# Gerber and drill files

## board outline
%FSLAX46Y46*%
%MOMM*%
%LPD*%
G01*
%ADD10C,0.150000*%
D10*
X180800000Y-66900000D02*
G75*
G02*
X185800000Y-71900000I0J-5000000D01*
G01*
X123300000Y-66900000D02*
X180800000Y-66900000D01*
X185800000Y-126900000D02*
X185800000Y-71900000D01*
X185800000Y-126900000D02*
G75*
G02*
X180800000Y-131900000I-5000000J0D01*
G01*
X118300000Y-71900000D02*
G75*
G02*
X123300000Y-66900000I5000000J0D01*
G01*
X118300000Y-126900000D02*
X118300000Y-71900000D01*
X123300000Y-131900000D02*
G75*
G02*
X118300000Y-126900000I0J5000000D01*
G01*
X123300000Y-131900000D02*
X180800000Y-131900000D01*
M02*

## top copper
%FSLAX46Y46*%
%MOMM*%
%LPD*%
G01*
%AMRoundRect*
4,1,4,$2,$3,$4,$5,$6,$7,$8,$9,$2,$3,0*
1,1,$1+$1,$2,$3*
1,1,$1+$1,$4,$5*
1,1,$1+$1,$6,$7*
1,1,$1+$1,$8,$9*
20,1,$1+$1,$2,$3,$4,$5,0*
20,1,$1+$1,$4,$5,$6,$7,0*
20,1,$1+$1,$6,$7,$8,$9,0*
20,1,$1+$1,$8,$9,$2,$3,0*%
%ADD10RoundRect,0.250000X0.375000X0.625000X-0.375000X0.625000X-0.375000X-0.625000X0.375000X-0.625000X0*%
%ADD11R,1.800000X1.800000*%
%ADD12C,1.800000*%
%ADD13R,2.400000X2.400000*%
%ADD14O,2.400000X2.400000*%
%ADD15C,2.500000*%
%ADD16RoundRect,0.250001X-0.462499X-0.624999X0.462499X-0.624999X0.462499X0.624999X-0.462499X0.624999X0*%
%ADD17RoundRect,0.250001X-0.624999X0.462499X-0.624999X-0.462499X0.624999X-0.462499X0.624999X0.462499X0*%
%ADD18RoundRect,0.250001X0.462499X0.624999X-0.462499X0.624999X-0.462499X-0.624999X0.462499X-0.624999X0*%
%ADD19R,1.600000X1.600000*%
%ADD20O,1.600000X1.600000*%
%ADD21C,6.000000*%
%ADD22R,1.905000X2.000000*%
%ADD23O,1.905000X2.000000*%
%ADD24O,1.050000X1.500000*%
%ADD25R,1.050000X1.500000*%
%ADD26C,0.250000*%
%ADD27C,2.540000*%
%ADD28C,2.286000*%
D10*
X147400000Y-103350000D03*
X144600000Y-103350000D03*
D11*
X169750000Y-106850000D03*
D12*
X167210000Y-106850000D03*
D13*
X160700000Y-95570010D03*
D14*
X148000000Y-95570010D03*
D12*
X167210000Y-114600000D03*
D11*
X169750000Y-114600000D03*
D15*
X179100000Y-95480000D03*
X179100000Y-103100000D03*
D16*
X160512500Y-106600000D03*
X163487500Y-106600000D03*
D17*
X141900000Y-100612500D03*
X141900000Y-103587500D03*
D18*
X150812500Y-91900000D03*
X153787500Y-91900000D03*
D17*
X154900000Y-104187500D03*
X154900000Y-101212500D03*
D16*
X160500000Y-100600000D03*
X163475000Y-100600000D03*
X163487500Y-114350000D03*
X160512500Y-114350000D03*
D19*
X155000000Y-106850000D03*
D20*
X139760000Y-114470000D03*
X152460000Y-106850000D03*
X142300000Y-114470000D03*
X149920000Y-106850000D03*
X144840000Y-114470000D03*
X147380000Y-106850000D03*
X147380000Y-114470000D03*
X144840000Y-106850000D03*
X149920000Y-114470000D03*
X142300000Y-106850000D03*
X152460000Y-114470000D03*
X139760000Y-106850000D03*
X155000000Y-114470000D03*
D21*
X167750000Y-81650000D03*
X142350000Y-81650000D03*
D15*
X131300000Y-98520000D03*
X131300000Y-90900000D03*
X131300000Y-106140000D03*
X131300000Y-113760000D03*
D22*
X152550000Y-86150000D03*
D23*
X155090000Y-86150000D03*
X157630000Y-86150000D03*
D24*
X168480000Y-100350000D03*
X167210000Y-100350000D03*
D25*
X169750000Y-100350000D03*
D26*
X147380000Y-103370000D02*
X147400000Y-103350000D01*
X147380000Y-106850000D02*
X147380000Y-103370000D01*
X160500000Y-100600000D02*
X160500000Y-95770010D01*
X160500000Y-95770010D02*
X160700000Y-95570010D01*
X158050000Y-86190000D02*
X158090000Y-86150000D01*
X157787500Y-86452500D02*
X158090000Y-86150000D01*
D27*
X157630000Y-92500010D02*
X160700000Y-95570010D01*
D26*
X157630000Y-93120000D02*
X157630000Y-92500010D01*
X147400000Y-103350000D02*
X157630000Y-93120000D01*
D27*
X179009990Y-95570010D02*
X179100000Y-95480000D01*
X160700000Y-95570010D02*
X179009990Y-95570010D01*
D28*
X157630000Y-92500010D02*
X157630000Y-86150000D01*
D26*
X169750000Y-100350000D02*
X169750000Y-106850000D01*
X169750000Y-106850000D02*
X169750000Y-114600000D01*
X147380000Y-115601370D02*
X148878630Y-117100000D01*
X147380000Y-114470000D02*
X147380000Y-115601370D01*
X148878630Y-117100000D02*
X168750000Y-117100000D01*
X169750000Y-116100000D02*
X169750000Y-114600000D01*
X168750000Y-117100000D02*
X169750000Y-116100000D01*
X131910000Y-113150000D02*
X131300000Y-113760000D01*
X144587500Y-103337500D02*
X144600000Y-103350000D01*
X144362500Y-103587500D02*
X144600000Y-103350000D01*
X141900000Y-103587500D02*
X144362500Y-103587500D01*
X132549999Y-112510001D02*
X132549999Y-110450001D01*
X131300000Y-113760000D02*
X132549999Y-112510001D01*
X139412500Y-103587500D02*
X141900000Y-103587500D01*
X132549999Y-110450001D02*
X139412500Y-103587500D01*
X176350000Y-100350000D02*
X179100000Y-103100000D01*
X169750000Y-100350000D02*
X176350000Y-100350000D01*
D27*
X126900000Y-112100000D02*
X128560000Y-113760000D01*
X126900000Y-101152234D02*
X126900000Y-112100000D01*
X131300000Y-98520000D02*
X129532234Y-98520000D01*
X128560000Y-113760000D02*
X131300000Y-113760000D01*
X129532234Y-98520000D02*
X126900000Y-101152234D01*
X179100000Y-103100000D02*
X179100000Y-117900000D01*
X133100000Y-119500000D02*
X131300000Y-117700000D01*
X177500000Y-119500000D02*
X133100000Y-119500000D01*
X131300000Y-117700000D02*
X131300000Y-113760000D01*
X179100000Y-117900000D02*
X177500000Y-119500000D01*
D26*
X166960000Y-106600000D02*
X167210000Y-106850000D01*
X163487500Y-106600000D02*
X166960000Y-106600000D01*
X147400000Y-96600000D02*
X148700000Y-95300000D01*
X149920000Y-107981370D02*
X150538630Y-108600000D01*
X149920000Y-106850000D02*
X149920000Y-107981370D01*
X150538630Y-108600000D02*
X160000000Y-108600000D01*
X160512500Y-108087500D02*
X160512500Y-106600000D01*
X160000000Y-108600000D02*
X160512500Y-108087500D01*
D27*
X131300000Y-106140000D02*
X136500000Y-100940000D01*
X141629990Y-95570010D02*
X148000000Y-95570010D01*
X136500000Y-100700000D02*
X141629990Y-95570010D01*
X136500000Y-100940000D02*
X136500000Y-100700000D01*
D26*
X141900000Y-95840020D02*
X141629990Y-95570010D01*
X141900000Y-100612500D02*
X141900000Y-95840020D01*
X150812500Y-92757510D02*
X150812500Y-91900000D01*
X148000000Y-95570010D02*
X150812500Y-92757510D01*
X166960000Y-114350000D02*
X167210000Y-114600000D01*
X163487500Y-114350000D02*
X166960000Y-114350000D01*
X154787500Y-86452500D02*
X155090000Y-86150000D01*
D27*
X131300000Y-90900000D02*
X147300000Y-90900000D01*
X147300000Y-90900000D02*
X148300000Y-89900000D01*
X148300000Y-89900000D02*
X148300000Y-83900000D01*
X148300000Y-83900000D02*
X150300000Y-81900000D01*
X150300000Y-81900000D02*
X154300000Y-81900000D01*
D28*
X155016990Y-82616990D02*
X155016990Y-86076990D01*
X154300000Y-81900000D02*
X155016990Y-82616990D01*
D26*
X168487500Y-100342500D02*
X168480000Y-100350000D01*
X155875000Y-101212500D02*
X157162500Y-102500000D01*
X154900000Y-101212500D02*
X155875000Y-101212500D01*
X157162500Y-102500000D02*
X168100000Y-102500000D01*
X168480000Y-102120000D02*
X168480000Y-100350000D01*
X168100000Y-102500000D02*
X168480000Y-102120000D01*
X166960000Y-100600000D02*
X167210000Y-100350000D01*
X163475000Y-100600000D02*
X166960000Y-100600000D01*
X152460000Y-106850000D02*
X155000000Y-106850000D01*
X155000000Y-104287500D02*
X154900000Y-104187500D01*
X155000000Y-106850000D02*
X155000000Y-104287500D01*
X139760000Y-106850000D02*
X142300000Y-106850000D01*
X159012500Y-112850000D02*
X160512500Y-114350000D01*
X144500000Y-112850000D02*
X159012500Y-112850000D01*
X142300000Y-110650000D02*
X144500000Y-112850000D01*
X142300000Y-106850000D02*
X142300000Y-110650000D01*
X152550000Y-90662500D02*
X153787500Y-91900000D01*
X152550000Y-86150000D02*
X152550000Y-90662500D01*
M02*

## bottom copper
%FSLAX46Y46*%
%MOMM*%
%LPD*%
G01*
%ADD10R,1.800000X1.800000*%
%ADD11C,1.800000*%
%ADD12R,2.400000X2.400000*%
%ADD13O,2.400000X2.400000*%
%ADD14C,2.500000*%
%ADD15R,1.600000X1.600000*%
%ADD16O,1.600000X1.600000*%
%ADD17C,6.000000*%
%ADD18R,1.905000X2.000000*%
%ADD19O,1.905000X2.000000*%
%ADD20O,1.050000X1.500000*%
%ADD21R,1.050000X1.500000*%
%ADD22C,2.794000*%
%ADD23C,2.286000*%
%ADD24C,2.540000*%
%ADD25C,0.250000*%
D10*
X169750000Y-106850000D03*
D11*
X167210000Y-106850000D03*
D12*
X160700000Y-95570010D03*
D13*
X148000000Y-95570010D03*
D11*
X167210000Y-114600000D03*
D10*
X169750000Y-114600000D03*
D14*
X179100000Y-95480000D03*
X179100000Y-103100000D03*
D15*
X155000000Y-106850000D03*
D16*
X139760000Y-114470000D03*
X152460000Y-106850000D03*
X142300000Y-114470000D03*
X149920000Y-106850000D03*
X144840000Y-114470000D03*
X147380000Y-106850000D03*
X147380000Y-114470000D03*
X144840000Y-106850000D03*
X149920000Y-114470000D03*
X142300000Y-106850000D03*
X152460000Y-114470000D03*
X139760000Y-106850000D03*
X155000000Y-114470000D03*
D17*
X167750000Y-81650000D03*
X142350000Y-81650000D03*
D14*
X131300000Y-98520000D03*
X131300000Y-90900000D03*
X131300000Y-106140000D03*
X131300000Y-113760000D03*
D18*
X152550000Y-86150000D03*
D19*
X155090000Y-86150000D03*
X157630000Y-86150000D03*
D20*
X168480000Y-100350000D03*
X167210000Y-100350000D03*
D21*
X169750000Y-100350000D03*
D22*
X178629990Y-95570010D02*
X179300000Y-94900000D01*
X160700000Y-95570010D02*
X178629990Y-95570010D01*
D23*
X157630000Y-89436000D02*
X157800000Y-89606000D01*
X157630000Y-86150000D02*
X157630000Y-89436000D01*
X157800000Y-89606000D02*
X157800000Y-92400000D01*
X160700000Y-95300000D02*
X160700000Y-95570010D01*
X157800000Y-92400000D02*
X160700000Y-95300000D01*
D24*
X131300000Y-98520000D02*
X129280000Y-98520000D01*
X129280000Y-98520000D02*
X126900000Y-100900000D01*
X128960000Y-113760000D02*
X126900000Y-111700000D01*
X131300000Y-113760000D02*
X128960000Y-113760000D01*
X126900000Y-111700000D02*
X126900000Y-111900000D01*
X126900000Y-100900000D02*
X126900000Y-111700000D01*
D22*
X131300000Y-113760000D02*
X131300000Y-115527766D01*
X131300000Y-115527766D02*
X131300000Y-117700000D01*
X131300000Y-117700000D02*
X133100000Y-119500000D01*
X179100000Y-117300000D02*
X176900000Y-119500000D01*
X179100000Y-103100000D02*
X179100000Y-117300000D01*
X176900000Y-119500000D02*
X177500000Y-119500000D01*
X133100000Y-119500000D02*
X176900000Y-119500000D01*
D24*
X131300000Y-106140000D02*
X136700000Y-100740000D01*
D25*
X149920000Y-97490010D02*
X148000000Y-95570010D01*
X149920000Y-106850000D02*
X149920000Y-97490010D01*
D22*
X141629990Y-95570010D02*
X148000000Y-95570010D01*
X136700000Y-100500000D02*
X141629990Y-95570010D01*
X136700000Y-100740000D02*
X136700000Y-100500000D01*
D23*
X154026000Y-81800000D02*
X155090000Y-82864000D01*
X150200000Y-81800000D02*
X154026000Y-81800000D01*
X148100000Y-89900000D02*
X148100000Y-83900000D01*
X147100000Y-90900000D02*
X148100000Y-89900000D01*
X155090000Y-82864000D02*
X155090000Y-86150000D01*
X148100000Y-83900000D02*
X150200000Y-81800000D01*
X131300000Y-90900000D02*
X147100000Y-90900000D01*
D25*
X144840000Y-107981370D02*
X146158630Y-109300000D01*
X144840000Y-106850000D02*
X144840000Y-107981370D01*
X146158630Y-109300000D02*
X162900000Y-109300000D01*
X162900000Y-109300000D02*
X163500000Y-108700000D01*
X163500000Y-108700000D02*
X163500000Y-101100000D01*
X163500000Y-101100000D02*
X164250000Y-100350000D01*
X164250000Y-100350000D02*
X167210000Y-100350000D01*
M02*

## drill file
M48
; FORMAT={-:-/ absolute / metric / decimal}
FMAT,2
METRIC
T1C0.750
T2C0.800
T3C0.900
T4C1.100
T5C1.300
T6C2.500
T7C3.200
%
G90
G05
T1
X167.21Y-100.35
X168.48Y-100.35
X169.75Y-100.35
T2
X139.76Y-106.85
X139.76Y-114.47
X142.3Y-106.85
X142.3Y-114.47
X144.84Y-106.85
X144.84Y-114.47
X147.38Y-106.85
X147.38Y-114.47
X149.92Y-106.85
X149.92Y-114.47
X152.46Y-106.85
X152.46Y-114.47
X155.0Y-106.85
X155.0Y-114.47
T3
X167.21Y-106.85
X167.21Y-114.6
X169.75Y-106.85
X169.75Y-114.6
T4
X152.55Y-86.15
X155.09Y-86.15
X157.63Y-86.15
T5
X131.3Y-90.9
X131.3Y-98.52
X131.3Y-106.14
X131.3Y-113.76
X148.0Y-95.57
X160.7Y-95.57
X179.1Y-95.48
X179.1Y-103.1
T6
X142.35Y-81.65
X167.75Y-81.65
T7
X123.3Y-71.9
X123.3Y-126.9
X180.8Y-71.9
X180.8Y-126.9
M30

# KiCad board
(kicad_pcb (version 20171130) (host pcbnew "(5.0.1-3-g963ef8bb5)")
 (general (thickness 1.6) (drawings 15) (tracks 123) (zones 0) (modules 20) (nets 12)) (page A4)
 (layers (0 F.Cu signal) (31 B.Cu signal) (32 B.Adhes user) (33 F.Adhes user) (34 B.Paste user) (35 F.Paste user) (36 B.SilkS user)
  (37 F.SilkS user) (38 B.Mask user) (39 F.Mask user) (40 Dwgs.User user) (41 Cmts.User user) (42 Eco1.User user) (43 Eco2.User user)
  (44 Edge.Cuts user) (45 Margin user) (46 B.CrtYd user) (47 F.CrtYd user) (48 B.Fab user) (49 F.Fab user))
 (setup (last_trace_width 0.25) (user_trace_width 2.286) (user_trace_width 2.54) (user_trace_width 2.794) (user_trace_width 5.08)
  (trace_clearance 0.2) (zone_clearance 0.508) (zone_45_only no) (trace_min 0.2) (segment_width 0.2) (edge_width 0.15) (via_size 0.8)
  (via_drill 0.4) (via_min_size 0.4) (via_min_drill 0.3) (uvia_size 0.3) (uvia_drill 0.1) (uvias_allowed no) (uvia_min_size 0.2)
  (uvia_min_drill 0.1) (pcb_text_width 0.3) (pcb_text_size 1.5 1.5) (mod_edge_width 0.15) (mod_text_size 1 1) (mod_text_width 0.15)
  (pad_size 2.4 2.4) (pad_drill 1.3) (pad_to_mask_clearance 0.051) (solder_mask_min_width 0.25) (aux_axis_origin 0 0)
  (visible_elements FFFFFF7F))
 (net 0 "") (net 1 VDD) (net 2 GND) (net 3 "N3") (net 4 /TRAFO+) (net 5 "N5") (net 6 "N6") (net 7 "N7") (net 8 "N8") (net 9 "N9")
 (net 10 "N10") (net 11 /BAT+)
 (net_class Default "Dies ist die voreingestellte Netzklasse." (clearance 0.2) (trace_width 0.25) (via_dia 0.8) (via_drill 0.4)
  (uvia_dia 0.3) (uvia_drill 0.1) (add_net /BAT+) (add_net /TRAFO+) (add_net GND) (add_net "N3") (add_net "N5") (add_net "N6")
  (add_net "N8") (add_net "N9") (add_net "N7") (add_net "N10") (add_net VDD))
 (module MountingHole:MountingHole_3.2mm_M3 (layer F.Cu) (at 180.8 126.9)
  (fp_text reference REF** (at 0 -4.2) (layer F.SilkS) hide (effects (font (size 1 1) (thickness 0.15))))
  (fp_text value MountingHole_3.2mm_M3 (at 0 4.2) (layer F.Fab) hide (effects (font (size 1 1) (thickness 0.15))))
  (pad 1 np_thru_hole circle (at 0 0) (size 3.2 3.2) (drill 3.2) (layers *.Cu *.Mask)))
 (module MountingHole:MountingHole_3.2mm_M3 (layer F.Cu) (at 180.8 71.9)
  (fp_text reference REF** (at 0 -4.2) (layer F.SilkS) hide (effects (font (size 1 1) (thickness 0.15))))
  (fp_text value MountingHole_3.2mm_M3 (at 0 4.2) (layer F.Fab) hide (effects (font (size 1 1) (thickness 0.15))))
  (pad 1 np_thru_hole circle (at 0 0) (size 3.2 3.2) (drill 3.2) (layers *.Cu *.Mask)))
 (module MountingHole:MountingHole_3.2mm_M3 (layer F.Cu) (at 123.3 71.9)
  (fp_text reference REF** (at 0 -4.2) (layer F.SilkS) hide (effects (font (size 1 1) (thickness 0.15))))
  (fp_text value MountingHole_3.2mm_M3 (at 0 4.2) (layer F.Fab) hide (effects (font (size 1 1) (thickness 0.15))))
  (pad 1 np_thru_hole circle (at 0 0) (size 3.2 3.2) (drill 3.2) (layers *.Cu *.Mask)))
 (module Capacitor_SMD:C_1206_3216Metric (layer F.Cu) (at 146 103.35 180)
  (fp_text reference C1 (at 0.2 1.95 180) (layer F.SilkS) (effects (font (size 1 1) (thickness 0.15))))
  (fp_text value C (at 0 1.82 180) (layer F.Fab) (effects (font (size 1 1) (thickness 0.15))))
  (pad 1 smd roundrect (at -1.4 0 180) (size 1.25 1.75) (layers F.Cu F.Paste F.Mask) (roundrect_rratio 0.2) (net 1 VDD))
  (pad 2 smd roundrect (at 1.4 0 180) (size 1.25 1.75) (layers F.Cu F.Paste F.Mask) (roundrect_rratio 0.2) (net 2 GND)))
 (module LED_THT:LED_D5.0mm (layer F.Cu) (at 169.75 106.85 180)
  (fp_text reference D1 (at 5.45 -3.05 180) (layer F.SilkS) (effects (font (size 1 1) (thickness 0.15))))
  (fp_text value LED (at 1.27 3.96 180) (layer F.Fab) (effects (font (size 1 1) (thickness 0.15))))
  (pad 1 thru_hole rect (at 0 0 180) (size 1.8 1.8) (drill 0.9) (layers *.Cu *.Mask) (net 2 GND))
  (pad 2 thru_hole circle (at 2.54 0 180) (size 1.8 1.8) (drill 0.9) (layers *.Cu *.Mask) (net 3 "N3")))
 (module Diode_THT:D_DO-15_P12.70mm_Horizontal (layer F.Cu) (at 160.7 95.57001 180)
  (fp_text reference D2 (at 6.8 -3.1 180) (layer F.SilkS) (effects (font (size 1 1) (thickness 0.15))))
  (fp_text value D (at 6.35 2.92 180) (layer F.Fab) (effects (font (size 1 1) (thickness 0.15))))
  (pad 1 thru_hole rect (at 0 0 180) (size 2.4 2.4) (drill 1.3) (layers *.Cu *.Mask) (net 1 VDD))
  (pad 2 thru_hole oval (at 12.7 0 180) (size 2.4 2.4) (drill 1.3) (layers *.Cu *.Mask) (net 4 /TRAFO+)))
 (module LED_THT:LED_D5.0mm (layer F.Cu) (at 169.75 114.6 180)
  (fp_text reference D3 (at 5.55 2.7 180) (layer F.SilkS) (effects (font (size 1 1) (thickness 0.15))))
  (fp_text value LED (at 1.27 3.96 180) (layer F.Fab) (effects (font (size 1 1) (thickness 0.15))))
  (pad 2 thru_hole circle (at 2.54 0 180) (size 1.8 1.8) (drill 0.9) (layers *.Cu *.Mask) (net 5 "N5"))
  (pad 1 thru_hole rect (at 0 0 180) (size 1.8 1.8) (drill 0.9) (layers *.Cu *.Mask) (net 2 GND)))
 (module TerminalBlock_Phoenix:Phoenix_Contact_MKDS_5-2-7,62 (layer F.Cu) (at 179.1 103.1 90)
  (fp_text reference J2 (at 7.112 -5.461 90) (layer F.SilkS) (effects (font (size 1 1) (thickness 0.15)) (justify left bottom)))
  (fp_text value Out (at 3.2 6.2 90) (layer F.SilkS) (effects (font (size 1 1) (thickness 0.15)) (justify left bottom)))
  (pad 2 thru_hole circle (at 7.62 0 90) (size 2.5 2.5) (drill 1.3) (layers *.Cu *.Mask) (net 1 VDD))
  (pad 1 thru_hole circle (at 0 0 90) (size 2.5 2.5) (drill 1.3) (layers *.Cu *.Mask) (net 2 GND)))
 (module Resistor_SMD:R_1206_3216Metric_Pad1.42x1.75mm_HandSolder (layer F.Cu) (at 162 106.6)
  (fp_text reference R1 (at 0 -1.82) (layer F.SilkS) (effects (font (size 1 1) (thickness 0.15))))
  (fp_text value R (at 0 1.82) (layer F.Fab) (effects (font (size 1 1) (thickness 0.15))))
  (pad 1 smd roundrect (at -1.4875 0) (size 1.425 1.75) (layers F.Cu F.Paste F.Mask) (roundrect_rratio 0.175439) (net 4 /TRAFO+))
  (pad 2 smd roundrect (at 1.4875 0) (size 1.425 1.75) (layers F.Cu F.Paste F.Mask) (roundrect_rratio 0.175439) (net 3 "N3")))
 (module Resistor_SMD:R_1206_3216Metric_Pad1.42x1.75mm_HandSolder (layer F.Cu) (at 141.9 102.1 270)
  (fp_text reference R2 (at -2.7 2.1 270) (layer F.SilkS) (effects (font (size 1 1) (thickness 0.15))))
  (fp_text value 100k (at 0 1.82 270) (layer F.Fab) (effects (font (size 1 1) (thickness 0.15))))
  (pad 1 smd roundrect (at -1.4875 0 270) (size 1.425 1.75) (layers F.Cu F.Paste F.Mask) (roundrect_rratio 0.175439) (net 4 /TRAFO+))
  (pad 2 smd roundrect (at 1.4875 0 270) (size 1.425 1.75) (layers F.Cu F.Paste F.Mask) (roundrect_rratio 0.175439) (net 2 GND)))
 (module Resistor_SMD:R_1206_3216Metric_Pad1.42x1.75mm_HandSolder (layer F.Cu) (at 152.3 91.9 180)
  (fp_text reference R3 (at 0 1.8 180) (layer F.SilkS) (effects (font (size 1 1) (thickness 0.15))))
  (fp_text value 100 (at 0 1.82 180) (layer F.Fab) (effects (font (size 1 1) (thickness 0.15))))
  (pad 2 smd roundrect (at 1.4875 0 180) (size 1.425 1.75) (layers F.Cu F.Paste F.Mask) (roundrect_rratio 0.175439) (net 4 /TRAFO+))
  (pad 1 smd roundrect (at -1.4875 0 180) (size 1.425 1.75) (layers F.Cu F.Paste F.Mask) (roundrect_rratio 0.175439) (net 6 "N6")))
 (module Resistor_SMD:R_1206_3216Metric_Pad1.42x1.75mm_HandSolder (layer F.Cu) (at 154.9 102.7 270)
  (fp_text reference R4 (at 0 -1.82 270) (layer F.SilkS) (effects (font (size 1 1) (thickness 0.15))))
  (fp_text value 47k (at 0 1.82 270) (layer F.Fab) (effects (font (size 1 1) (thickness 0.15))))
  (pad 2 smd roundrect (at 1.4875 0 270) (size 1.425 1.75) (layers F.Cu F.Paste F.Mask) (roundrect_rratio 0.175439) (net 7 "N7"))
  (pad 1 smd roundrect (at -1.4875 0 270) (size 1.425 1.75) (layers F.Cu F.Paste F.Mask) (roundrect_rratio 0.175439) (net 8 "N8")))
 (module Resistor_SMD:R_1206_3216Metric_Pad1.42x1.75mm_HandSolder (layer F.Cu) (at 161.9875 100.6)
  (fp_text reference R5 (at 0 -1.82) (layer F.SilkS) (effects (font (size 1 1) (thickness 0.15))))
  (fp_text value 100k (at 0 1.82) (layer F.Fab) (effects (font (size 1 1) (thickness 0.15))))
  (pad 1 smd roundrect (at -1.4875 0) (size 1.425 1.75) (layers F.Cu F.Paste F.Mask) (roundrect_rratio 0.175439) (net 1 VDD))
  (pad 2 smd roundrect (at 1.4875 0) (size 1.425 1.75) (layers F.Cu F.Paste F.Mask) (roundrect_rratio 0.175439) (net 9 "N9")))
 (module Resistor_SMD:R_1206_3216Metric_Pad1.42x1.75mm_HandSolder (layer F.Cu) (at 162 114.35)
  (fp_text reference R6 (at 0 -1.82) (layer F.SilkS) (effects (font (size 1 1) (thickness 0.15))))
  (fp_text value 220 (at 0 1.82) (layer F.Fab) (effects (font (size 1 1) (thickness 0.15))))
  (pad 2 smd roundrect (at 1.4875 0) (size 1.425 1.75) (layers F.Cu F.Paste F.Mask) (roundrect_rratio 0.175439) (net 5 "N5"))
  (pad 1 smd roundrect (at -1.4875 0) (size 1.425 1.75) (layers F.Cu F.Paste F.Mask) (roundrect_rratio 0.175439) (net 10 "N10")))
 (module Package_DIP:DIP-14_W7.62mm (layer F.Cu) (at 155 106.85 270)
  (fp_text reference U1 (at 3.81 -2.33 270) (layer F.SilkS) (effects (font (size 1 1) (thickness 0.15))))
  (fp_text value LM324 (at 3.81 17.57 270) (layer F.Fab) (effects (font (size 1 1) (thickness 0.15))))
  (pad 1 thru_hole rect (at 0 0 270) (size 1.6 1.6) (drill 0.8) (layers *.Cu *.Mask) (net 7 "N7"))
  (pad 8 thru_hole oval (at 7.62 15.24 270) (size 1.6 1.6) (drill 0.8) (layers *.Cu *.Mask))
  (pad 2 thru_hole oval (at 0 2.54 270) (size 1.6 1.6) (drill 0.8) (layers *.Cu *.Mask) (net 7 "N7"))
  (pad 9 thru_hole oval (at 7.62 12.7 270) (size 1.6 1.6) (drill 0.8) (layers *.Cu *.Mask))
  (pad 3 thru_hole oval (at 0 5.08 270) (size 1.6 1.6) (drill 0.8) (layers *.Cu *.Mask) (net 4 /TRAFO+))
  (pad 10 thru_hole oval (at 7.62 10.16 270) (size 1.6 1.6) (drill 0.8) (layers *.Cu *.Mask))
  (pad 4 thru_hole oval (at 0 7.62 270) (size 1.6 1.6) (drill 0.8) (layers *.Cu *.Mask) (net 1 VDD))
  (pad 11 thru_hole oval (at 7.62 7.62 270) (size 1.6 1.6) (drill 0.8) (layers *.Cu *.Mask) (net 2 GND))
  (pad 5 thru_hole oval (at 0 10.16 270) (size 1.6 1.6) (drill 0.8) (layers *.Cu *.Mask) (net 9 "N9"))
  (pad 12 thru_hole oval (at 7.62 5.08 270) (size 1.6 1.6) (drill 0.8) (layers *.Cu *.Mask))
  (pad 6 thru_hole oval (at 0 12.7 270) (size 1.6 1.6) (drill 0.8) (layers *.Cu *.Mask) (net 10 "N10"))
  (pad 13 thru_hole oval (at 7.62 2.54 270) (size 1.6 1.6) (drill 0.8) (layers *.Cu *.Mask))
  (pad 7 thru_hole oval (at 0 15.24 270) (size 1.6 1.6) (drill 0.8) (layers *.Cu *.Mask) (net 10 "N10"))
  (pad 14 thru_hole oval (at 7.62 0 270) (size 1.6 1.6) (drill 0.8) (layers *.Cu *.Mask)))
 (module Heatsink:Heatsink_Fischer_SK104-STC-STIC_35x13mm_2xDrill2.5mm (layer F.Cu) (at 155.05 81.65)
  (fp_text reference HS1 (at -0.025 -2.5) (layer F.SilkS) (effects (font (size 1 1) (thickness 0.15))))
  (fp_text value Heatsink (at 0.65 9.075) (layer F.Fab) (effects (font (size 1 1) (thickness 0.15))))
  (pad 1 thru_hole circle (at 12.7 0) (size 6 6) (drill 2.5) (layers *.Cu *.Mask))
  (pad 1 thru_hole circle (at -12.7 0 180) (size 6 6) (drill 2.5) (layers *.Cu *.Mask)))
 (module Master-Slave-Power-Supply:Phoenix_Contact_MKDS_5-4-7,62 (layer F.Cu) (at 131.3 90.9 270)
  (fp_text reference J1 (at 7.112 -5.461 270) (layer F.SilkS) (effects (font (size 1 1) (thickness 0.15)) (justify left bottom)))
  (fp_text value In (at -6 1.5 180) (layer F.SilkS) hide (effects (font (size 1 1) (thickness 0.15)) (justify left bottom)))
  (pad 2 thru_hole circle (at 7.62 0 270) (size 2.5 2.5) (drill 1.3) (layers *.Cu *.Mask) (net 2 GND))
  (pad 1 thru_hole circle (at 0 0 270) (size 2.5 2.5) (drill 1.3) (layers *.Cu *.Mask) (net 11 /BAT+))
  (pad 3 thru_hole circle (at 15.24 0 270) (size 2.5 2.5) (drill 1.3) (layers *.Cu *.Mask) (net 4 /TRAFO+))
  (pad 4 thru_hole circle (at 22.86 0 270) (size 2.5 2.5) (drill 1.3) (layers *.Cu *.Mask) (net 2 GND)))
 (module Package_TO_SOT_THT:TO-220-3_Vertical (layer F.Cu) (at 152.55 86.15)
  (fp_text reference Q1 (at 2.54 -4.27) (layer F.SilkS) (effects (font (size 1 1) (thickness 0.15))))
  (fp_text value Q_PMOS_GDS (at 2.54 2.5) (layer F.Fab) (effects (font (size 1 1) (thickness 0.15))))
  (pad 1 thru_hole rect (at 0 0) (size 1.905 2) (drill 1.1) (layers *.Cu *.Mask) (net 6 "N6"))
  (pad 2 thru_hole oval (at 2.54 0) (size 1.905 2) (drill 1.1) (layers *.Cu *.Mask) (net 11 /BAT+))
  (pad 3 thru_hole oval (at 5.08 0) (size 1.905 2) (drill 1.1) (layers *.Cu *.Mask) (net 1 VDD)))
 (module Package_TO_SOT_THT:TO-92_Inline (layer F.Cu) (at 169.75 100.35 180)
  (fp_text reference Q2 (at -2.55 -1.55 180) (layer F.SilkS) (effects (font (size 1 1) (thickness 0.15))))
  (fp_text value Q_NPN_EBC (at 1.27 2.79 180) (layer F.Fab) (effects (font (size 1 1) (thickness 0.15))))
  (pad 2 thru_hole oval (at 1.27 0 180) (size 1.05 1.5) (drill 0.75) (layers *.Cu *.Mask) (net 8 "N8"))
  (pad 3 thru_hole oval (at 2.54 0 180) (size 1.05 1.5) (drill 0.75) (layers *.Cu *.Mask) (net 9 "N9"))
  (pad 1 thru_hole rect (at 0 0 180) (size 1.05 1.5) (drill 0.75) (layers *.Cu *.Mask) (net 2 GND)))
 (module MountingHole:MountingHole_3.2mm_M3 (layer F.Cu) (at 123.3 126.9)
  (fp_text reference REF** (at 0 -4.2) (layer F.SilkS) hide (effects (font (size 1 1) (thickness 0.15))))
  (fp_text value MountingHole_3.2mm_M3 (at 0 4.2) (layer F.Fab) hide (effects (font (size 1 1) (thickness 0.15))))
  (pad 1 np_thru_hole circle (at 0 0) (size 3.2 3.2) (drill 3.2) (layers *.Cu *.Mask)))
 (gr_arc (start 180.8 71.9) (end 185.8 71.9) (angle -90) (layer Edge.Cuts) (width 0.15))
 (gr_line (start 123.3 66.9) (end 180.8 66.9) (layer Edge.Cuts) (width 0.15))
 (gr_line (start 185.8 126.9) (end 185.8 71.9) (layer Edge.Cuts) (width 0.15))
 (gr_arc (start 180.8 126.9) (end 180.8 131.9) (angle -90) (layer Edge.Cuts) (width 0.15))
 (gr_arc (start 123.3 71.9) (end 123.3 66.9) (angle -90) (layer Edge.Cuts) (width 0.15))
 (gr_line (start 118.3 126.9) (end 118.3 71.9) (layer Edge.Cuts) (width 0.15))
 (gr_arc (start 123.3 126.9) (end 118.3 126.9) (angle -90) (layer Edge.Cuts) (width 0.15))
 (gr_line (start 123.3 131.9) (end 180.8 131.9) (layer Edge.Cuts) (width 0.15))
 (segment (start 147.38 103.37) (end 147.4 103.35) (width 0.25) (layer F.Cu) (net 1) (status 30))
 (segment (start 147.38 106.85) (end 147.38 103.37) (width 0.25) (layer F.Cu) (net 1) (status 30))
 (segment (start 160.5 100.6) (end 160.5 95.77001) (width 0.25) (layer F.Cu) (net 1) (status 10))
 (segment (start 160.5 95.77001) (end 160.7 95.57001) (width 0.25) (layer F.Cu) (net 1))
 (segment (start 158.05 86.19) (end 158.09 86.15) (width 0.25) (layer F.Cu) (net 1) (status 30))
 (segment (start 157.7875 86.4525) (end 158.09 86.15) (width 0.25) (layer F.Cu) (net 1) (status 30))
 (segment (start 157.63 92.50001) (end 160.7 95.57001) (width 2.54) (layer F.Cu) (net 1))
 (segment (start 157.63 93.12) (end 157.63 92.50001) (width 0.25) (layer F.Cu) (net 1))
 (segment (start 147.4 103.35) (end 157.63 93.12) (width 0.25) (layer F.Cu) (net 1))
 (segment (start 179.00999 95.57001) (end 179.1 95.48) (width 2.54) (layer F.Cu) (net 1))
 (segment (start 160.7 95.57001) (end 179.00999 95.57001) (width 2.54) (layer F.Cu) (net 1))
 (segment (start 178.62999 95.57001) (end 179.3 94.9) (width 2.794) (layer B.Cu) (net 1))
 (segment (start 160.7 95.57001) (end 178.62999 95.57001) (width 2.794) (layer B.Cu) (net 1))
 (segment (start 157.63 89.436) (end 157.8 89.606) (width 2.286) (layer B.Cu) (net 1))
 (segment (start 157.63 86.15) (end 157.63 89.436) (width 2.286) (layer B.Cu) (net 1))
 (segment (start 157.8 89.606) (end 157.8 92.4) (width 2.286) (layer B.Cu) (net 1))
 (segment (start 160.7 95.3) (end 160.7 95.57001) (width 2.286) (layer B.Cu) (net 1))
 (segment (start 157.8 92.4) (end 160.7 95.3) (width 2.286) (layer B.Cu) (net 1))
 (segment (start 157.63 92.50001) (end 157.63 86.15) (width 2.286) (layer F.Cu) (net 1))
 (segment (start 169.75 100.35) (end 169.75 106.85) (width 0.25) (layer F.Cu) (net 2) (status 30))
 (segment (start 169.75 106.85) (end 169.75 114.6) (width 0.25) (layer F.Cu) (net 2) (status 30))
 (segment (start 147.38 115.60137) (end 148.87863 117.1) (width 0.25) (layer F.Cu) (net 2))
 (segment (start 147.38 114.47) (end 147.38 115.60137) (width 0.25) (layer F.Cu) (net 2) (status 10))
 (segment (start 148.87863 117.1) (end 168.75 117.1) (width 0.25) (layer F.Cu) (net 2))
 (segment (start 169.75 116.1) (end 169.75 114.6) (width 0.25) (layer F.Cu) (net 2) (status 20))
 (segment (start 168.75 117.1) (end 169.75 116.1) (width 0.25) (layer F.Cu) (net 2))
 (segment (start 131.91 113.15) (end 131.3 113.76) (width 0.25) (layer F.Cu) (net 2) (status 30))
 (segment (start 144.5875 103.3375) (end 144.6 103.35) (width 0.25) (layer F.Cu) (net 2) (status 30))
 (segment (start 144.3625 103.5875) (end 144.6 103.35) (width 0.25) (layer F.Cu) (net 2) (status 30))
 (segment (start 141.9 103.5875) (end 144.3625 103.5875) (width 0.25) (layer F.Cu) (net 2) (status 30))
 (segment (start 132.549999 112.510001) (end 132.549999 110.450001) (width 0.25) (layer F.Cu) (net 2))
 (segment (start 131.3 113.76) (end 132.549999 112.510001) (width 0.25) (layer F.Cu) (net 2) (status 10))
 (segment (start 139.4125 103.5875) (end 141.9 103.5875) (width 0.25) (layer F.Cu) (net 2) (status 20))
 (segment (start 132.549999 110.450001) (end 139.4125 103.5875) (width 0.25) (layer F.Cu) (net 2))
 (segment (start 176.35 100.35) (end 179.1 103.1) (width 0.25) (layer F.Cu) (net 2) (status 20))
 (segment (start 169.75 100.35) (end 176.35 100.35) (width 0.25) (layer F.Cu) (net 2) (status 10))
 (segment (start 126.9 112.1) (end 128.56 113.76) (width 2.54) (layer F.Cu) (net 2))
 (segment (start 126.9 101.152234) (end 126.9 112.1) (width 2.54) (layer F.Cu) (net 2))
 (segment (start 131.3 98.52) (end 129.532234 98.52) (width 2.54) (layer F.Cu) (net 2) (status 10))
 (segment (start 131.3 98.52) (end 129.28 98.52) (width 2.54) (layer B.Cu) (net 2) (status 10))
 (segment (start 128.56 113.76) (end 131.3 113.76) (width 2.54) (layer F.Cu) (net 2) (status 20))
 (segment (start 129.532234 98.52) (end 126.9 101.152234) (width 2.54) (layer F.Cu) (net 2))
 (segment (start 129.28 98.52) (end 126.9 100.9) (width 2.54) (layer B.Cu) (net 2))
 (segment (start 128.96 113.76) (end 126.9 111.7) (width 2.54) (layer B.Cu) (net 2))
 (segment (start 131.3 113.76) (end 128.96 113.76) (width 2.54) (layer B.Cu) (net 2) (status 10))
 (segment (start 126.9 111.7) (end 126.9 111.9) (width 2.54) (layer B.Cu) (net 2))
 (segment (start 126.9 100.9) (end 126.9 111.7) (width 2.54) (layer B.Cu) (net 2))
 (segment (start 179.1 103.1) (end 179.1 117.9) (width 2.54) (layer F.Cu) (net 2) (status 10))
 (segment (start 133.1 119.5) (end 131.3 117.7) (width 2.54) (layer F.Cu) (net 2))
 (segment (start 131.3 113.76) (end 131.3 115.527766) (width 2.794) (layer B.Cu) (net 2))
 (segment (start 177.5 119.5) (end 133.1 119.5) (width 2.54) (layer F.Cu) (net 2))
 (segment (start 131.3 117.7) (end 131.3 113.76) (width 2.54) (layer F.Cu) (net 2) (status 20))
 (segment (start 179.1 117.9) (end 177.5 119.5) (width 2.54) (layer F.Cu) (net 2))
 (segment (start 131.3 115.527766) (end 131.3 117.7) (width 2.794) (layer B.Cu) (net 2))
 (segment (start 131.3 117.7) (end 133.1 119.5) (width 2.794) (layer B.Cu) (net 2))
 (segment (start 179.1 117.3) (end 176.9 119.5) (width 2.794) (layer B.Cu) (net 2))
 (segment (start 179.1 103.1) (end 179.1 117.3) (width 2.794) (layer B.Cu) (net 2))
 (segment (start 176.9 119.5) (end 177.5 119.5) (width 2.794) (layer B.Cu) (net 2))
 (segment (start 133.1 119.5) (end 176.9 119.5) (width 2.794) (layer B.Cu) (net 2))
 (segment (start 166.96 106.6) (end 167.21 106.85) (width 0.25) (layer F.Cu) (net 3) (status 30))
 (segment (start 163.4875 106.6) (end 166.96 106.6) (width 0.25) (layer F.Cu) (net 3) (status 30))
 (segment (start 147.4 96.6) (end 148.7 95.3) (width 0.25) (layer F.Cu) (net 4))
 (segment (start 149.92 107.98137) (end 150.53863 108.6) (width 0.25) (layer F.Cu) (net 4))
 (segment (start 149.92 106.85) (end 149.92 107.98137) (width 0.25) (layer F.Cu) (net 4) (status 10))
 (segment (start 150.53863 108.6) (end 160 108.6) (width 0.25) (layer F.Cu) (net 4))
 (segment (start 160.5125 108.0875) (end 160.5125 106.6) (width 0.25) (layer F.Cu) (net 4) (status 20))
 (segment (start 160 108.6) (end 160.5125 108.0875) (width 0.25) (layer F.Cu) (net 4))
 (segment (start 131.3 106.14) (end 136.5 100.94) (width 2.54) (layer F.Cu) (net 4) (status 10))
 (segment (start 131.3 106.14) (end 136.7 100.74) (width 2.54) (layer B.Cu) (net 4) (status 10))
 (segment (start 141.62999 95.57001) (end 148 95.57001) (width 2.54) (layer F.Cu) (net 4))
 (segment (start 136.5 100.7) (end 141.62999 95.57001) (width 2.54) (layer F.Cu) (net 4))
 (segment (start 136.5 100.94) (end 136.5 100.7) (width 2.54) (layer F.Cu) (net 4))
 (segment (start 149.92 97.49001) (end 148 95.57001) (width 0.25) (layer B.Cu) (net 4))
 (segment (start 149.92 106.85) (end 149.92 97.49001) (width 0.25) (layer B.Cu) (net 4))
 (segment (start 141.9 95.84002) (end 141.62999 95.57001) (width 0.25) (layer F.Cu) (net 4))
 (segment (start 141.9 100.6125) (end 141.9 95.84002) (width 0.25) (layer F.Cu) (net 4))
 (segment (start 141.62999 95.57001) (end 148 95.57001) (width 2.794) (layer B.Cu) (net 4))
 (segment (start 136.7 100.5) (end 141.62999 95.57001) (width 2.794) (layer B.Cu) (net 4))
 (segment (start 136.7 100.74) (end 136.7 100.5) (width 2.794) (layer B.Cu) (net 4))
 (segment (start 150.8125 92.75751) (end 150.8125 91.9) (width 0.25) (layer F.Cu) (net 4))
 (segment (start 148 95.57001) (end 150.8125 92.75751) (width 0.25) (layer F.Cu) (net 4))
 (segment (start 166.96 114.35) (end 167.21 114.6) (width 0.25) (layer F.Cu) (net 5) (status 30))
 (segment (start 163.4875 114.35) (end 166.96 114.35) (width 0.25) (layer F.Cu) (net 5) (status 30))
 (segment (start 154.7875 86.4525) (end 155.09 86.15) (width 0.25) (layer F.Cu) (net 11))
 (segment (start 131.3 90.9) (end 147.3 90.9) (width 2.54) (layer F.Cu) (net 11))
 (segment (start 147.3 90.9) (end 148.3 89.9) (width 2.54) (layer F.Cu) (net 11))
 (segment (start 148.3 89.9) (end 148.3 83.9) (width 2.54) (layer F.Cu) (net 11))
 (segment (start 148.3 83.9) (end 150.3 81.9) (width 2.54) (layer F.Cu) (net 11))
 (segment (start 150.3 81.9) (end 154.3 81.9) (width 2.54) (layer F.Cu) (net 11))
 (segment (start 155.01699 82.61699) (end 155.01699 86.07699) (width 2.286) (layer F.Cu) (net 11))
 (segment (start 154.3 81.9) (end 155.01699 82.61699) (width 2.286) (layer F.Cu) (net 11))
 (segment (start 154.026 81.8) (end 155.09 82.864) (width 2.286) (layer B.Cu) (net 11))
 (segment (start 150.2 81.8) (end 154.026 81.8) (width 2.286) (layer B.Cu) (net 11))
 (segment (start 148.1 89.9) (end 148.1 83.9) (width 2.286) (layer B.Cu) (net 11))
 (segment (start 147.1 90.9) (end 148.1 89.9) (width 2.286) (layer B.Cu) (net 11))
 (segment (start 155.09 82.864) (end 155.09 86.15) (width 2.286) (layer B.Cu) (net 11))
 (segment (start 148.1 83.9) (end 150.2 81.8) (width 2.286) (layer B.Cu) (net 11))
 (segment (start 131.3 90.9) (end 147.1 90.9) (width 2.286) (layer B.Cu) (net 11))
 (segment (start 168.4875 100.3425) (end 168.48 100.35) (width 0.25) (layer F.Cu) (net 8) (status 30))
 (segment (start 155.875 101.2125) (end 157.1625 102.5) (width 0.25) (layer F.Cu) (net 8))
 (segment (start 154.9 101.2125) (end 155.875 101.2125) (width 0.25) (layer F.Cu) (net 8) (status 10))
 (segment (start 157.1625 102.5) (end 168.1 102.5) (width 0.25) (layer F.Cu) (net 8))
 (segment (start 168.48 102.12) (end 168.48 100.35) (width 0.25) (layer F.Cu) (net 8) (status 20))
 (segment (start 168.1 102.5) (end 168.48 102.12) (width 0.25) (layer F.Cu) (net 8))
 (segment (start 166.96 100.6) (end 167.21 100.35) (width 0.25) (layer F.Cu) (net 9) (status 30))
 (segment (start 163.475 100.6) (end 166.96 100.6) (width 0.25) (layer F.Cu) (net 9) (status 30))
 (segment (start 144.84 107.98137) (end 146.15863 109.3) (width 0.25) (layer B.Cu) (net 9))
 (segment (start 144.84 106.85) (end 144.84 107.98137) (width 0.25) (layer B.Cu) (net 9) (status 10))
 (segment (start 146.15863 109.3) (end 162.9 109.3) (width 0.25) (layer B.Cu) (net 9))
 (segment (start 162.9 109.3) (end 163.5 108.7) (width 0.25) (layer B.Cu) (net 9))
 (segment (start 163.5 108.7) (end 163.5 101.1) (width 0.25) (layer B.Cu) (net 9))
 (segment (start 163.5 101.1) (end 164.25 100.35) (width 0.25) (layer B.Cu) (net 9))
 (segment (start 164.25 100.35) (end 167.21 100.35) (width 0.25) (layer B.Cu) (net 9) (status 20))
 (segment (start 152.46 106.85) (end 155 106.85) (width 0.25) (layer F.Cu) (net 7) (status 30))
 (segment (start 155 104.2875) (end 154.9 104.1875) (width 0.25) (layer F.Cu) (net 7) (status 30))
 (segment (start 155 106.85) (end 155 104.2875) (width 0.25) (layer F.Cu) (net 7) (status 30))
 (segment (start 139.76 106.85) (end 142.3 106.85) (width 0.25) (layer F.Cu) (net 10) (status 30))
 (segment (start 159.0125 112.85) (end 160.5125 114.35) (width 0.25) (layer F.Cu) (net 10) (status 20))
 (segment (start 144.5 112.85) (end 159.0125 112.85) (width 0.25) (layer F.Cu) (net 10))
 (segment (start 142.3 110.65) (end 144.5 112.85) (width 0.25) (layer F.Cu) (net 10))
 (segment (start 142.3 106.85) (end 142.3 110.65) (width 0.25) (layer F.Cu) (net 10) (status 10))
 (segment (start 152.55 90.6625) (end 153.7875 91.9) (width 0.25) (layer F.Cu) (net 6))
 (segment (start 152.55 86.15) (end 152.55 90.6625) (width 0.25) (layer F.Cu) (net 6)))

